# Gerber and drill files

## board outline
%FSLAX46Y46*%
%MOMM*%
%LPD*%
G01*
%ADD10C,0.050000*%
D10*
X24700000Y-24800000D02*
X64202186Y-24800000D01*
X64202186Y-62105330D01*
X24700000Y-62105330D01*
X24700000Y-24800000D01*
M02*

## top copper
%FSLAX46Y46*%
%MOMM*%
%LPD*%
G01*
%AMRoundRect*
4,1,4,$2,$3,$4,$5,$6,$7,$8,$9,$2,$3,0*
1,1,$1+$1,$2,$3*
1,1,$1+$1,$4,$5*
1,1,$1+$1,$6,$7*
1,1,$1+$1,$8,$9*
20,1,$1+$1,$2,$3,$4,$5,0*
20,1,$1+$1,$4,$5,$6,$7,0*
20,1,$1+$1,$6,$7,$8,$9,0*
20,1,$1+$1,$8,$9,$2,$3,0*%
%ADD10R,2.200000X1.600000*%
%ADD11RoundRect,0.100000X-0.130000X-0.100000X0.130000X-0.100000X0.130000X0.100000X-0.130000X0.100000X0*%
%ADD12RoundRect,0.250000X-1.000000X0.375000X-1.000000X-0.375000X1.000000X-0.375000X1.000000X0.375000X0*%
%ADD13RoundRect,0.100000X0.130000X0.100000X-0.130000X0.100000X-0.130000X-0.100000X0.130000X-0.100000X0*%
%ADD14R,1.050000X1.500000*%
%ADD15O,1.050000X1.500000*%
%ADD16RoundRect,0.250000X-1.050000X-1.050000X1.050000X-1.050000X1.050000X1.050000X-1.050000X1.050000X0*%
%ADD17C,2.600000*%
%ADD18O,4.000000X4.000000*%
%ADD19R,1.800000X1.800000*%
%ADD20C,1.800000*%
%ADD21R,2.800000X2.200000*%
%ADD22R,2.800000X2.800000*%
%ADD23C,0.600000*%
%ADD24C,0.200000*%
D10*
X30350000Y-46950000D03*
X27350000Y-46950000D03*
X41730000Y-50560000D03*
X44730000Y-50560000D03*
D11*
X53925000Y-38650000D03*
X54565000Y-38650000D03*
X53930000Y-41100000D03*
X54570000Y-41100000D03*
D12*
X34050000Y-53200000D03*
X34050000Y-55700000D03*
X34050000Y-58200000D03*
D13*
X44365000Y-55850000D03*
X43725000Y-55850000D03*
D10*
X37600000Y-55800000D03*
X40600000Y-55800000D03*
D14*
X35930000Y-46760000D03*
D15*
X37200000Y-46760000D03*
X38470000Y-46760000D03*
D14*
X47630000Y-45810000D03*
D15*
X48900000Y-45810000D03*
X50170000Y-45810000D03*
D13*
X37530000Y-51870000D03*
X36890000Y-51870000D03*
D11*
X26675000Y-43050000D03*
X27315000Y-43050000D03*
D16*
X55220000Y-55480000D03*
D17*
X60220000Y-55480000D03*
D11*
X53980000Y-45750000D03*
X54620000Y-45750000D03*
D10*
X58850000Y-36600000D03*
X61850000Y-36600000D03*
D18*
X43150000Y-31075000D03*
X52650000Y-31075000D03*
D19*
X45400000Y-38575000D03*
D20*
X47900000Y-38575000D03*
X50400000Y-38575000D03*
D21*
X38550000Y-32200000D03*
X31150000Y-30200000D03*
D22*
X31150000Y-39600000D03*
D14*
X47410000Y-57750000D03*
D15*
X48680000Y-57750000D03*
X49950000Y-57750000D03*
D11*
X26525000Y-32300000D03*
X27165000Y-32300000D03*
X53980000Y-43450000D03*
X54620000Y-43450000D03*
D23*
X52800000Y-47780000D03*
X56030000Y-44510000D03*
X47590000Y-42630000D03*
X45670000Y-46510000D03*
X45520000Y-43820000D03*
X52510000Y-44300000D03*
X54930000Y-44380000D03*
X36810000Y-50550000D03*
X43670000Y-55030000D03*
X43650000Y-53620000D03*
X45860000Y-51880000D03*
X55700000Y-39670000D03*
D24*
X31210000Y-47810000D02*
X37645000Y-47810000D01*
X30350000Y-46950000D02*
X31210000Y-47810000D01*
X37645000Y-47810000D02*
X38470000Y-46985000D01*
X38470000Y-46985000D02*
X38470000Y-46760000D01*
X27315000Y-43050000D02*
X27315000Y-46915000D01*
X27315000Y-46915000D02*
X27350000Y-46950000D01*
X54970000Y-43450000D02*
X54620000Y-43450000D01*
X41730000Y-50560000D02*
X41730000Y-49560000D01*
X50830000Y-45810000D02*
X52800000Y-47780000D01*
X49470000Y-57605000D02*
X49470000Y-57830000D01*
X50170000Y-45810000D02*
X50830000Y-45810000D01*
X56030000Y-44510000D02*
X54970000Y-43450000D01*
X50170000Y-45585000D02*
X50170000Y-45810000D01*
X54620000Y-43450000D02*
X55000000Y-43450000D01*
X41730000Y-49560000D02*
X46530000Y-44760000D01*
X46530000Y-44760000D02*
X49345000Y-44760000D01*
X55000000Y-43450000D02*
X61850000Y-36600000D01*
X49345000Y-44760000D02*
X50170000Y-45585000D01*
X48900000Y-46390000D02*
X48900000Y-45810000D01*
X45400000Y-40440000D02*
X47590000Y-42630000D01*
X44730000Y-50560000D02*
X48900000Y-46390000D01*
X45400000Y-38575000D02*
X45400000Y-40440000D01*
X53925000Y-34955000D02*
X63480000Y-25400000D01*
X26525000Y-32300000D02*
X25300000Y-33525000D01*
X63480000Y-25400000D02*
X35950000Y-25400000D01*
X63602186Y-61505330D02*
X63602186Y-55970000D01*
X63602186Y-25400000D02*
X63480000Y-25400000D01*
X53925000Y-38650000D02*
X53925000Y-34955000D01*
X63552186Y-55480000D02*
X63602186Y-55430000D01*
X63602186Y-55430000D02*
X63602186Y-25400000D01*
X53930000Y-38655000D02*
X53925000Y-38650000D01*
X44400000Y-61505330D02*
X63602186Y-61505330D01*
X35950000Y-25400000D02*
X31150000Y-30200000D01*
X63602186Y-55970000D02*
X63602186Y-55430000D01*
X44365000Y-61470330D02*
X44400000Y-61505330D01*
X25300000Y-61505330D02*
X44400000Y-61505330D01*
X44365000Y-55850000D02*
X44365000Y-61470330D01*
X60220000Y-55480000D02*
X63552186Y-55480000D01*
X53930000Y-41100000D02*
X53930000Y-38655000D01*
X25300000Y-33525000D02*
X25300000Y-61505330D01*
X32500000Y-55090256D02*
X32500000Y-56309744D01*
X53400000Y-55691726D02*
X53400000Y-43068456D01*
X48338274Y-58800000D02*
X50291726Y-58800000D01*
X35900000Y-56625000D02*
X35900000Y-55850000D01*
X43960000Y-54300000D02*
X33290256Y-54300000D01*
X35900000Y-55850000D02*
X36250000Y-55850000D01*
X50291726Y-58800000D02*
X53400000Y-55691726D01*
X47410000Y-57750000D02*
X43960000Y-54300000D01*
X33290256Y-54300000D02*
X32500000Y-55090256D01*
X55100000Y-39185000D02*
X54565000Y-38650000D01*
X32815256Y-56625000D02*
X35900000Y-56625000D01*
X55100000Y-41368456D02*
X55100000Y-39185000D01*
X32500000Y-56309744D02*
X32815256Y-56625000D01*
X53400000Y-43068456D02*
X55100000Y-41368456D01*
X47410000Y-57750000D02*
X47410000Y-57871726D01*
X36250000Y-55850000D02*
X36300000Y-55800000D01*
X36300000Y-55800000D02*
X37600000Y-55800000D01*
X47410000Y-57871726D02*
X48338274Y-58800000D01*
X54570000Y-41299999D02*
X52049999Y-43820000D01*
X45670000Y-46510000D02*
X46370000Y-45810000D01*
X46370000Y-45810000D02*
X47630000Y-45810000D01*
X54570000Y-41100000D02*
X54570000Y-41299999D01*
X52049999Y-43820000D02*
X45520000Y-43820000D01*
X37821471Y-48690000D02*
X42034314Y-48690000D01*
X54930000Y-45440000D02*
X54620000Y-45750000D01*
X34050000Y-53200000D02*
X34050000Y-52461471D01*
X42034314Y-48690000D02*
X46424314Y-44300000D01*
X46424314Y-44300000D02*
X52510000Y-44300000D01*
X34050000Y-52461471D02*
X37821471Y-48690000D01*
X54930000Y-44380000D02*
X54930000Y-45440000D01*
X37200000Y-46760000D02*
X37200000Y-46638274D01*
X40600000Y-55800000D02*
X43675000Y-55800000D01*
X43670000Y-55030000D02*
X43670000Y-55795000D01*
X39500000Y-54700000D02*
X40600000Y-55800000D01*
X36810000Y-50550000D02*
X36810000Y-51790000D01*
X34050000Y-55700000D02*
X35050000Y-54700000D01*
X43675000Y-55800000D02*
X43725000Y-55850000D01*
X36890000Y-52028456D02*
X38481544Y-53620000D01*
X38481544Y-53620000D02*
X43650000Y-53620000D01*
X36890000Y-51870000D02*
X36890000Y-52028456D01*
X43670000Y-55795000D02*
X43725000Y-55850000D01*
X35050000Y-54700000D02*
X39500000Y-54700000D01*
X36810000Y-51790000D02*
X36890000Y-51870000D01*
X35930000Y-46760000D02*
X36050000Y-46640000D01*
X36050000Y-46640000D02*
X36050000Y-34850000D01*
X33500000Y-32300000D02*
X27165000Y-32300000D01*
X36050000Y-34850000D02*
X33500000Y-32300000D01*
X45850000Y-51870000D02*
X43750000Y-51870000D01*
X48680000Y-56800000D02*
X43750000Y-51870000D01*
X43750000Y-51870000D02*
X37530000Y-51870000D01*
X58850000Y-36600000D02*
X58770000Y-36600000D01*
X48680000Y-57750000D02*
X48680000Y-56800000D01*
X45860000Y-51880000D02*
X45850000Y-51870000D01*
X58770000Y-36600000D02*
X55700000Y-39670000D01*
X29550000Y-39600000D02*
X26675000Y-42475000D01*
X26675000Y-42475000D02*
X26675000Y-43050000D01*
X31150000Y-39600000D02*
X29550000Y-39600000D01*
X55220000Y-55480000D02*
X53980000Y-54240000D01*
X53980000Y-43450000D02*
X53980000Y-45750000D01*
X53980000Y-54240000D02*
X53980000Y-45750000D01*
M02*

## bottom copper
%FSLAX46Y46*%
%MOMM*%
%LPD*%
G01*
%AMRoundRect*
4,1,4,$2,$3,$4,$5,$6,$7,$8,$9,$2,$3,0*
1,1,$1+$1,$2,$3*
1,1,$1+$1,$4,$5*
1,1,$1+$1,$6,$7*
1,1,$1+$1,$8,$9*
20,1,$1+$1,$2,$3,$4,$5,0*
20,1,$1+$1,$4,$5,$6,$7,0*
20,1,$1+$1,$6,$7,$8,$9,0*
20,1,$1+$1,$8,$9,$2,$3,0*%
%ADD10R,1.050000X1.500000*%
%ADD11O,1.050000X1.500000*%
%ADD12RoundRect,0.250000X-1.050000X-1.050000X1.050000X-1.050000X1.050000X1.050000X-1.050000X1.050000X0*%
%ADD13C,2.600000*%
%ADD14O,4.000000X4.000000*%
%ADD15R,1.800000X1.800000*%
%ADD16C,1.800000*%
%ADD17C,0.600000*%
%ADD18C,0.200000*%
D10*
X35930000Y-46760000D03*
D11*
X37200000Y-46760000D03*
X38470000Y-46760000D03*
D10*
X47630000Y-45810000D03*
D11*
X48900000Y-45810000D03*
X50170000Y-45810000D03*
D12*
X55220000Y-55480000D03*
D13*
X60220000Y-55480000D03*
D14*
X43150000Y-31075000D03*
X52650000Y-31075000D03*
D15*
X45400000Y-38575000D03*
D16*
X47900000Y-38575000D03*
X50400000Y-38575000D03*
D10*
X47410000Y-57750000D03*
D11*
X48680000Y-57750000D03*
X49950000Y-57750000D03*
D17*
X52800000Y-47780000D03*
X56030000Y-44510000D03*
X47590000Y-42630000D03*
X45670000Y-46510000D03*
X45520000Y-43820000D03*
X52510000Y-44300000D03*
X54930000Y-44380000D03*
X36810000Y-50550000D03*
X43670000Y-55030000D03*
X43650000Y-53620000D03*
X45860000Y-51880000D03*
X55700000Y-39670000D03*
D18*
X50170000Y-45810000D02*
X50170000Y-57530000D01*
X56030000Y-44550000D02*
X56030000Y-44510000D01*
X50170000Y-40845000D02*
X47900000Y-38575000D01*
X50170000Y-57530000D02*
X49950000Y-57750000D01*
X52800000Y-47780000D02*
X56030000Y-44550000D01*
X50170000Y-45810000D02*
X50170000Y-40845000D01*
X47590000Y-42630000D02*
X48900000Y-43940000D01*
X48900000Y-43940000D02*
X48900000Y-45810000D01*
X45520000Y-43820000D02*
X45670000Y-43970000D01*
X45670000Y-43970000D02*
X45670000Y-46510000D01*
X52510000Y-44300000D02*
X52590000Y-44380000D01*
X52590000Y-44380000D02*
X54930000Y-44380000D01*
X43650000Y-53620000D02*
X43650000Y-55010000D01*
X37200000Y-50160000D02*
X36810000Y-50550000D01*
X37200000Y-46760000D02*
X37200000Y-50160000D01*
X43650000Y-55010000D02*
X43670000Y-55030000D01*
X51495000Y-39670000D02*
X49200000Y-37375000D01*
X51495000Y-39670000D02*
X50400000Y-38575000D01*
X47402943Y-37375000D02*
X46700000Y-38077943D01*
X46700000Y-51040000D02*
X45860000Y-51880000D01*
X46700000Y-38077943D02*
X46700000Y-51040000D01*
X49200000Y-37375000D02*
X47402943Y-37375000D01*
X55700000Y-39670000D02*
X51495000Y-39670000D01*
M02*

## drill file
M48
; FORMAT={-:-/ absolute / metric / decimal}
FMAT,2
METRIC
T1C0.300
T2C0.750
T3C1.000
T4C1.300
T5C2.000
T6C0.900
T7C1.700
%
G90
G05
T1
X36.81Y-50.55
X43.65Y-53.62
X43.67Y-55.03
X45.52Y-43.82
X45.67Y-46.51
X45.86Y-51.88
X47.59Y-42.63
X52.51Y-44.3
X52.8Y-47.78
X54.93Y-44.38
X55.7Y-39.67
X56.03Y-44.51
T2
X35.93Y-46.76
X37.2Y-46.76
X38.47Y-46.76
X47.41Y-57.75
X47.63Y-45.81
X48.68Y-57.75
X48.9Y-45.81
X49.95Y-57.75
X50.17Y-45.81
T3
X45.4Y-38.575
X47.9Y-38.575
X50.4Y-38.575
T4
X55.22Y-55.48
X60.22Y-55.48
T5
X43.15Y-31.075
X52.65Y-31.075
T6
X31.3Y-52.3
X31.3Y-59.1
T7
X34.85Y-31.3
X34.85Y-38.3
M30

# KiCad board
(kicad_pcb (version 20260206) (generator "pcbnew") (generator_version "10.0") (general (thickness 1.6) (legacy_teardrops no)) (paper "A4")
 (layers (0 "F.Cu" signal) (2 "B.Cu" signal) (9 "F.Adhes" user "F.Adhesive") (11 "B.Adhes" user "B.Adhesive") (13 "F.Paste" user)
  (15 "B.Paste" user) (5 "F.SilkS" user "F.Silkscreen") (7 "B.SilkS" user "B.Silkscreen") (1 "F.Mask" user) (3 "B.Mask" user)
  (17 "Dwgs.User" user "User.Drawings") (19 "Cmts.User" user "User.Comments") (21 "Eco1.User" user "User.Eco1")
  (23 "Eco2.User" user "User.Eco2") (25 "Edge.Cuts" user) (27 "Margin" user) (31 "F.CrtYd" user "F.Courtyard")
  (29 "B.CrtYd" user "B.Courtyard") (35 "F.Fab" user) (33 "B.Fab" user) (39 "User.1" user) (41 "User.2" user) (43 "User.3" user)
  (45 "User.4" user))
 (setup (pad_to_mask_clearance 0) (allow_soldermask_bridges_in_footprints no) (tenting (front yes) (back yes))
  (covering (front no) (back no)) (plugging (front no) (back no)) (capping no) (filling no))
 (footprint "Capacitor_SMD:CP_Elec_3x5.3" (layer "F.Cu") (at 28.85 46.95 180)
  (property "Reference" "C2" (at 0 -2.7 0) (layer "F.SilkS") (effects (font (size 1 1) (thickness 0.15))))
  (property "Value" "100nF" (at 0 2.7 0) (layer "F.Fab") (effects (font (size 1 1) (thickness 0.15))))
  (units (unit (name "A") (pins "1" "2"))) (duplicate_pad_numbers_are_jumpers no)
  (pad "1" smd rect (at -1.5 0 180) (size 2.2 1.6) (layers "F.Cu" "F.Mask" "F.Paste") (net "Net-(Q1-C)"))
  (pad "2" smd rect (at 1.5 0 180) (size 2.2 1.6) (layers "F.Cu" "F.Mask" "F.Paste") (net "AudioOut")))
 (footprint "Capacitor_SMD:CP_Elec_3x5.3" (layer "F.Cu") (at 43.23 50.56)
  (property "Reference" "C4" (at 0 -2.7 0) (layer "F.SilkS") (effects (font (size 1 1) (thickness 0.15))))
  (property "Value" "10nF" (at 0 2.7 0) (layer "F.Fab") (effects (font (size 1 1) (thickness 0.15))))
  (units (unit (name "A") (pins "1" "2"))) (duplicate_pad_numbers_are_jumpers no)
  (pad "1" smd rect (at -1.5 0) (size 2.2 1.6) (layers "F.Cu" "F.Mask" "F.Paste") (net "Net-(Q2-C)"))
  (pad "2" smd rect (at 1.5 0) (size 2.2 1.6) (layers "F.Cu" "F.Mask" "F.Paste") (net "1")))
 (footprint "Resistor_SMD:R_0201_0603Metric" (layer "F.Cu") (at 54.245 38.65)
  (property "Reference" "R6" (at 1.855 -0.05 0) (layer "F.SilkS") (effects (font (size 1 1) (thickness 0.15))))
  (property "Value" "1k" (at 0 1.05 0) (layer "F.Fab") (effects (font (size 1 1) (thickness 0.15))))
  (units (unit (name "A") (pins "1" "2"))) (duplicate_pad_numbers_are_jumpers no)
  (pad "" smd roundrect (at -0.345 0) (size 0.318 0.36) (layers "F.Paste") (roundrect_rratio 0.25))
  (pad "" smd roundrect (at 0.345 0) (size 0.318 0.36) (layers "F.Paste") (roundrect_rratio 0.25))
  (pad "1" smd roundrect (at -0.32 0) (size 0.46 0.4) (layers "F.Cu" "F.Mask") (roundrect_rratio 0.25) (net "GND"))
  (pad "2" smd roundrect (at 0.32 0) (size 0.46 0.4) (layers "F.Cu" "F.Mask") (roundrect_rratio 0.25) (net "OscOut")))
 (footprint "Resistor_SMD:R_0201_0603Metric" (layer "F.Cu") (at 54.25 41.1)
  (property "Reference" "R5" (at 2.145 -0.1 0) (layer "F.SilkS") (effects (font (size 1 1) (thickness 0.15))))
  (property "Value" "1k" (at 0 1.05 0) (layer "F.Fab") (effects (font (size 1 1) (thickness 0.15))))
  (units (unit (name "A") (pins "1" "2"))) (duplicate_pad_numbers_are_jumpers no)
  (pad "" smd roundrect (at -0.345 0) (size 0.318 0.36) (layers "F.Paste") (roundrect_rratio 0.25))
  (pad "" smd roundrect (at 0.345 0) (size 0.318 0.36) (layers "F.Paste") (roundrect_rratio 0.25))
  (pad "1" smd roundrect (at -0.32 0) (size 0.46 0.4) (layers "F.Cu" "F.Mask") (roundrect_rratio 0.25) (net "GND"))
  (pad "2" smd roundrect (at 0.32 0) (size 0.46 0.4) (layers "F.Cu" "F.Mask") (roundrect_rratio 0.25) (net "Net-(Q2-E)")))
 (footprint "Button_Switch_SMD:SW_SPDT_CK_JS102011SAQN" (layer "F.Cu") (at 31.3 55.7 -90)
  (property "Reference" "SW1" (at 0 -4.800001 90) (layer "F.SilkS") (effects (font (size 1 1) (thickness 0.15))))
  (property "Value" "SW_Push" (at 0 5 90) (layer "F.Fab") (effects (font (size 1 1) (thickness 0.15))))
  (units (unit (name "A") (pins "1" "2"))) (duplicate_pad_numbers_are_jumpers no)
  (pad "" np_thru_hole circle (at -3.4 0 270) (size 0.9 0.9) (drill 0.9) (layers "*.Cu" "*.Mask"))
  (pad "" np_thru_hole circle (at 3.4 0 270) (size 0.9 0.9) (drill 0.9) (layers "*.Cu" "*.Mask"))
  (pad "1" smd roundrect (at -2.5 -2.75 270) (size 1.25 2.5) (layers "F.Cu" "F.Mask" "F.Paste") (roundrect_rratio 0.2) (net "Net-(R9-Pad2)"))
  (pad "2" smd roundrect (at 0 -2.75 270) (size 1.25 2.5) (layers "F.Cu" "F.Mask" "F.Paste") (roundrect_rratio 0.2) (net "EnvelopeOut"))
  (pad "3" smd roundrect (at 2.5 -2.75 270) (size 1.25 2.5) (layers "F.Cu" "F.Mask" "F.Paste") (roundrect_rratio 0.2)))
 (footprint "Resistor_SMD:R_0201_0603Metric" (layer "F.Cu") (at 44.045 55.85 180)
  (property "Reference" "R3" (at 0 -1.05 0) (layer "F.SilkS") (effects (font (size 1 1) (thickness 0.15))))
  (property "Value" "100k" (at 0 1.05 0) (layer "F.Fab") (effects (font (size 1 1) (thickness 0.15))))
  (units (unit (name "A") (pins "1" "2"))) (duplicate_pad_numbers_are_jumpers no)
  (pad "" smd roundrect (at -0.345 0 180) (size 0.318 0.36) (layers "F.Paste") (roundrect_rratio 0.25))
  (pad "" smd roundrect (at 0.345 0 180) (size 0.318 0.36) (layers "F.Paste") (roundrect_rratio 0.25))
  (pad "1" smd roundrect (at -0.32 0 180) (size 0.46 0.4) (layers "F.Cu" "F.Mask") (roundrect_rratio 0.25) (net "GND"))
  (pad "2" smd roundrect (at 0.32 0 180) (size 0.46 0.4) (layers "F.Cu" "F.Mask") (roundrect_rratio 0.25) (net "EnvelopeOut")))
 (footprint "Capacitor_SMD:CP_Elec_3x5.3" (layer "F.Cu") (at 39.1 55.8)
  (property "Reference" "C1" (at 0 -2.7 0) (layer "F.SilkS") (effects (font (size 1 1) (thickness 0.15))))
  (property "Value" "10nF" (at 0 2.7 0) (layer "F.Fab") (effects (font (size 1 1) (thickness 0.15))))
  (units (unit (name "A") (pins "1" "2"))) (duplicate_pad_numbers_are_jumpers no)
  (pad "1" smd rect (at -1.5 0) (size 2.2 1.6) (layers "F.Cu" "F.Mask" "F.Paste") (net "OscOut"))
  (pad "2" smd rect (at 1.5 0) (size 2.2 1.6) (layers "F.Cu" "F.Mask" "F.Paste") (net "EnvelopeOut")))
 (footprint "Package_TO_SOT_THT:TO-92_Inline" (layer "F.Cu") (at 35.93 46.76)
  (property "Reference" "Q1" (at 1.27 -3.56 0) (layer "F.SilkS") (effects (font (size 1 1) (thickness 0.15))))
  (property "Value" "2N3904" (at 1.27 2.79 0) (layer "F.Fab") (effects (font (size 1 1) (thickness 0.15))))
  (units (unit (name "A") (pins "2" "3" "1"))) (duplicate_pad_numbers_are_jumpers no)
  (pad "1" thru_hole rect (at 0 0) (size 1.05 1.5) (drill 0.75) (layers "*.Cu" "*.Mask") (remove_unused_layers no) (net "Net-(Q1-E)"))
  (pad "2" thru_hole oval (at 1.27 0) (size 1.05 1.5) (drill 0.75) (layers "*.Cu" "*.Mask") (remove_unused_layers no) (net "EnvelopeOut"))
  (pad "3" thru_hole oval (at 2.54 0) (size 1.05 1.5) (drill 0.75) (layers "*.Cu" "*.Mask") (remove_unused_layers no) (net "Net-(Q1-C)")))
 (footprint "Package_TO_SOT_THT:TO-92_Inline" (layer "F.Cu") (at 47.63 45.81)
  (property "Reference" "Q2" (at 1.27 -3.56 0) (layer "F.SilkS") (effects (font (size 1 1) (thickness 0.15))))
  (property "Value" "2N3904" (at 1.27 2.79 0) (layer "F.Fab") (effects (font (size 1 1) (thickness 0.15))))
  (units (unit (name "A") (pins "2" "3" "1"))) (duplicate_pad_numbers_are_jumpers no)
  (pad "1" thru_hole rect (at 0 0) (size 1.05 1.5) (drill 0.75) (layers "*.Cu" "*.Mask") (remove_unused_layers no) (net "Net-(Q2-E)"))
  (pad "2" thru_hole oval (at 1.27 0) (size 1.05 1.5) (drill 0.75) (layers "*.Cu" "*.Mask") (remove_unused_layers no) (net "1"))
  (pad "3" thru_hole oval (at 2.54 0) (size 1.05 1.5) (drill 0.75) (layers "*.Cu" "*.Mask") (remove_unused_layers no) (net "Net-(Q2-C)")))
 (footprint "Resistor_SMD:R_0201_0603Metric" (layer "F.Cu") (at 37.21 51.87 180)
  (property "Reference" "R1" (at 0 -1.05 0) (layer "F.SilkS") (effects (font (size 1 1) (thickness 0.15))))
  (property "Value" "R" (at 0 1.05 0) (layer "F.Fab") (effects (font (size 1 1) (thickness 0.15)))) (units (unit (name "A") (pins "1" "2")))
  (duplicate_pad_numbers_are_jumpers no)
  (pad "" smd roundrect (at -0.345 0 180) (size 0.318 0.36) (layers "F.Paste") (roundrect_rratio 0.25))
  (pad "" smd roundrect (at 0.345 0 180) (size 0.318 0.36) (layers "F.Paste") (roundrect_rratio 0.25))
  (pad "1" smd roundrect (at -0.32 0 180) (size 0.46 0.4) (layers "F.Cu" "F.Mask") (roundrect_rratio 0.25) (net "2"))
  (pad "2" smd roundrect (at 0.32 0 180) (size 0.46 0.4) (layers "F.Cu" "F.Mask") (roundrect_rratio 0.25) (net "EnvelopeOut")))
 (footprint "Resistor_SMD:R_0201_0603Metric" (layer "F.Cu") (at 26.995 43.05)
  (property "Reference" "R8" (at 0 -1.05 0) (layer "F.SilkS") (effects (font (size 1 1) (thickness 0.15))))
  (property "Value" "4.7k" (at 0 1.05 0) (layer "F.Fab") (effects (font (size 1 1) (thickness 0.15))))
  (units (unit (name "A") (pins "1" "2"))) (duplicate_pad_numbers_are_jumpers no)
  (pad "" smd roundrect (at -0.345 0) (size 0.318 0.36) (layers "F.Paste") (roundrect_rratio 0.25))
  (pad "" smd roundrect (at 0.345 0) (size 0.318 0.36) (layers "F.Paste") (roundrect_rratio 0.25))
  (pad "1" smd roundrect (at -0.32 0) (size 0.46 0.4) (layers "F.Cu" "F.Mask") (roundrect_rratio 0.25) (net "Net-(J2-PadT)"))
  (pad "2" smd roundrect (at 0.32 0) (size 0.46 0.4) (layers "F.Cu" "F.Mask") (roundrect_rratio 0.25) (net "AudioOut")))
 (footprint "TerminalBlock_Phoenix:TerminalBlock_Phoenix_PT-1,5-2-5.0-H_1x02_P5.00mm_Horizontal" (layer "F.Cu") (at 55.22 55.48)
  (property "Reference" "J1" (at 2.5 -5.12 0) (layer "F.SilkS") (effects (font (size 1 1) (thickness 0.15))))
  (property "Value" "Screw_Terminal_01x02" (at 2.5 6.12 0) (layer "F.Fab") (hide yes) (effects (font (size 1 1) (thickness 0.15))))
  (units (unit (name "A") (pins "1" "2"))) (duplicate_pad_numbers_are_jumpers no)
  (pad "1" thru_hole roundrect (at 0 0) (size 2.6 2.6) (drill 1.3) (layers "*.Cu" "*.Mask") (remove_unused_layers no)
   (roundrect_rratio 0.096154) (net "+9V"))
  (pad "2" thru_hole circle (at 5 0) (size 2.6 2.6) (drill 1.3) (layers "*.Cu" "*.Mask") (remove_unused_layers no) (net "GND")))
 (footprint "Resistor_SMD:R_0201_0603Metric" (layer "F.Cu") (at 54.3 45.75)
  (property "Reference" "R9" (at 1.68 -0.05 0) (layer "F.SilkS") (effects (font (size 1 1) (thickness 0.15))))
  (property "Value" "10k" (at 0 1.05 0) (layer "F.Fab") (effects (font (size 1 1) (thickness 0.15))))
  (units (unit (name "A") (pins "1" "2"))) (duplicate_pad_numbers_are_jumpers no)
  (pad "" smd roundrect (at -0.345 0) (size 0.318 0.36) (layers "F.Paste") (roundrect_rratio 0.25))
  (pad "" smd roundrect (at 0.345 0) (size 0.318 0.36) (layers "F.Paste") (roundrect_rratio 0.25))
  (pad "1" smd roundrect (at -0.32 0) (size 0.46 0.4) (layers "F.Cu" "F.Mask") (roundrect_rratio 0.25) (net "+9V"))
  (pad "2" smd roundrect (at 0.32 0) (size 0.46 0.4) (layers "F.Cu" "F.Mask") (roundrect_rratio 0.25) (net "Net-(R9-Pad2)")))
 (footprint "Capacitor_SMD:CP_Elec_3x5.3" (layer "F.Cu") (at 60.35 36.6)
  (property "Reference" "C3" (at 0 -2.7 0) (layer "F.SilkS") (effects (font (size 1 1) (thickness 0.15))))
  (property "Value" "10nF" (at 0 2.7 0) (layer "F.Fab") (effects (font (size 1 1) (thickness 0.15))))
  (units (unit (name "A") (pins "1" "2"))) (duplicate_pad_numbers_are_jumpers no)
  (pad "1" smd rect (at -1.5 0) (size 2.2 1.6) (layers "F.Cu" "F.Mask" "F.Paste") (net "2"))
  (pad "2" smd rect (at 1.5 0) (size 2.2 1.6) (layers "F.Cu" "F.Mask" "F.Paste") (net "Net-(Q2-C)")))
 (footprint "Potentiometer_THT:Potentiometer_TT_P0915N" (layer "F.Cu") (at 45.4 38.575)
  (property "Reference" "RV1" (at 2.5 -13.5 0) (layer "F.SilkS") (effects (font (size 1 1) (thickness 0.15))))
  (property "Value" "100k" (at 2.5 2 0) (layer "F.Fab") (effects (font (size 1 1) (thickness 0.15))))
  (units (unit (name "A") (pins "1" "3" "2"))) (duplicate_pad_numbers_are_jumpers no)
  (pad "" thru_hole oval (at -2.25 -7.5) (size 4 4) (drill 2) (layers "*.Cu" "*.Mask") (remove_unused_layers no))
  (pad "" thru_hole oval (at 7.25 -7.5) (size 4 4) (drill 2) (layers "*.Cu" "*.Mask") (remove_unused_layers no))
  (pad "1" thru_hole rect (at 0 0) (size 1.8 1.8) (drill 1) (layers "*.Cu" "*.Mask") (remove_unused_layers no) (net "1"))
  (pad "2" thru_hole circle (at 2.5 0) (size 1.8 1.8) (drill 1) (layers "*.Cu" "*.Mask") (remove_unused_layers no) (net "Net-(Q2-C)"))
  (pad "3" thru_hole circle (at 5 0) (size 1.8 1.8) (drill 1) (layers "*.Cu" "*.Mask") (remove_unused_layers no) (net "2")))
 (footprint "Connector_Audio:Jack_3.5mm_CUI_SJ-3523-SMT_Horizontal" (layer "F.Cu") (at 34.85 33.8)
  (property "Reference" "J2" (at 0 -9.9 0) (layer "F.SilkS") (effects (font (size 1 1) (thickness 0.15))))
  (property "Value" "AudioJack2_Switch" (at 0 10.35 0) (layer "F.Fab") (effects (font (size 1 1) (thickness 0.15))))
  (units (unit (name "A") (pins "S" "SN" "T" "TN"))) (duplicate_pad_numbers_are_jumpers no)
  (pad "" np_thru_hole circle (at 0 -2.5) (size 1.7 1.7) (drill 1.7) (layers "*.Cu" "*.Mask"))
  (pad "" np_thru_hole circle (at 0 4.5) (size 1.7 1.7) (drill 1.7) (layers "*.Cu" "*.Mask"))
  (pad "R" smd rect (at 3.7 -1.6) (size 2.8 2.2) (layers "F.Cu" "F.Mask" "F.Paste"))
  (pad "S" smd rect (at -3.7 -3.6) (size 2.8 2.2) (layers "F.Cu" "F.Mask" "F.Paste") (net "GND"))
  (pad "T" smd rect (at -3.7 5.8) (size 2.8 2.8) (layers "F.Cu" "F.Mask" "F.Paste") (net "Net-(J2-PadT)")))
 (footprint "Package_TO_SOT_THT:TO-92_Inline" (layer "F.Cu") (at 47.41 57.75)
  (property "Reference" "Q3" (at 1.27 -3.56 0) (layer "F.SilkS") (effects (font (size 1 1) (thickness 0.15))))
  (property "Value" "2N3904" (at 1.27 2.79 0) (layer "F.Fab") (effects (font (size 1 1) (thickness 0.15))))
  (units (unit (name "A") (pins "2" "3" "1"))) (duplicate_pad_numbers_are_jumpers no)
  (pad "1" thru_hole rect (at 0 0) (size 1.05 1.5) (drill 0.75) (layers "*.Cu" "*.Mask") (remove_unused_layers no) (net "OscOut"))
  (pad "2" thru_hole oval (at 1.27 0) (size 1.05 1.5) (drill 0.75) (layers "*.Cu" "*.Mask") (remove_unused_layers no) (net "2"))
  (pad "3" thru_hole oval (at 2.54 0) (size 1.05 1.5) (drill 0.75) (layers "*.Cu" "*.Mask") (remove_unused_layers no) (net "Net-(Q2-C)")))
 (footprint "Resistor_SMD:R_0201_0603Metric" (layer "F.Cu") (at 26.845 32.3)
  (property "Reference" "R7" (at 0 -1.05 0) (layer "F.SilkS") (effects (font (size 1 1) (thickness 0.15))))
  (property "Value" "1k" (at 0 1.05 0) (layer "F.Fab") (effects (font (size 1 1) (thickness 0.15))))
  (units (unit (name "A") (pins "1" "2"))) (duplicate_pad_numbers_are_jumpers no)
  (pad "" smd roundrect (at -0.345 0) (size 0.318 0.36) (layers "F.Paste") (roundrect_rratio 0.25))
  (pad "" smd roundrect (at 0.345 0) (size 0.318 0.36) (layers "F.Paste") (roundrect_rratio 0.25))
  (pad "1" smd roundrect (at -0.32 0) (size 0.46 0.4) (layers "F.Cu" "F.Mask") (roundrect_rratio 0.25) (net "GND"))
  (pad "2" smd roundrect (at 0.32 0) (size 0.46 0.4) (layers "F.Cu" "F.Mask") (roundrect_rratio 0.25) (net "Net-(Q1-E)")))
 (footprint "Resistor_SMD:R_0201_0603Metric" (layer "F.Cu") (at 54.3 43.45)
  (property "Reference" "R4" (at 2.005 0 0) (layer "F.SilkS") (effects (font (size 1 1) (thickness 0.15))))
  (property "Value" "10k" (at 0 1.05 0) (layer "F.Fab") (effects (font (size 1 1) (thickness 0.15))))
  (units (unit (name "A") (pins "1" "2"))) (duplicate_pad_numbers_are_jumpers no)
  (pad "" smd roundrect (at -0.345 0) (size 0.318 0.36) (layers "F.Paste") (roundrect_rratio 0.25))
  (pad "" smd roundrect (at 0.345 0) (size 0.318 0.36) (layers "F.Paste") (roundrect_rratio 0.25))
  (pad "1" smd roundrect (at -0.32 0) (size 0.46 0.4) (layers "F.Cu" "F.Mask") (roundrect_rratio 0.25) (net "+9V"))
  (pad "2" smd roundrect (at 0.32 0) (size 0.46 0.4) (layers "F.Cu" "F.Mask") (roundrect_rratio 0.25) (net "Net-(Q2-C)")))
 (gr_rect (start 24.7 24.8) (end 64.202186 62.10533) (stroke (width 0.05) (type default)) (fill no) (layer "Edge.Cuts"))
 (segment (start 31.21 47.81) (end 37.645 47.81) (width 0.2) (layer "F.Cu") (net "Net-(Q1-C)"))
 (segment (start 30.35 46.95) (end 31.21 47.81) (width 0.2) (layer "F.Cu") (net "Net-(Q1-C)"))
 (segment (start 37.645 47.81) (end 38.47 46.985) (width 0.2) (layer "F.Cu") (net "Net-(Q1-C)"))
 (segment (start 38.47 46.985) (end 38.47 46.76) (width 0.2) (layer "F.Cu") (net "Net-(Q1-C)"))
 (segment (start 27.315 43.05) (end 27.315 46.915) (width 0.2) (layer "F.Cu") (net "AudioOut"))
 (segment (start 27.315 46.915) (end 27.35 46.95) (width 0.2) (layer "F.Cu") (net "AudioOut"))
 (segment (start 54.97 43.45) (end 54.62 43.45) (width 0.2) (layer "F.Cu") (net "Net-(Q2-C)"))
 (segment (start 41.73 50.56) (end 41.73 49.56) (width 0.2) (layer "F.Cu") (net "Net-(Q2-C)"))
 (segment (start 50.83 45.81) (end 52.8 47.78) (width 0.2) (layer "F.Cu") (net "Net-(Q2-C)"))
 (segment (start 49.47 57.605) (end 49.47 57.83) (width 0.2) (layer "F.Cu") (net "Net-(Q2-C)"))
 (segment (start 50.17 45.81) (end 50.83 45.81) (width 0.2) (layer "F.Cu") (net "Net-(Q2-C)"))
 (segment (start 56.03 44.51) (end 54.97 43.45) (width 0.2) (layer "F.Cu") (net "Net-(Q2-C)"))
 (segment (start 50.17 45.585) (end 50.17 45.81) (width 0.2) (layer "F.Cu") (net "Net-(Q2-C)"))
 (segment (start 54.62 43.45) (end 55 43.45) (width 0.2) (layer "F.Cu") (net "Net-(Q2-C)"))
 (segment (start 41.73 49.56) (end 46.53 44.76) (width 0.2) (layer "F.Cu") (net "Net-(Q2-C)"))
 (segment (start 46.53 44.76) (end 49.345 44.76) (width 0.2) (layer "F.Cu") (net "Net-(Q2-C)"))
 (segment (start 55 43.45) (end 61.85 36.6) (width 0.2) (layer "F.Cu") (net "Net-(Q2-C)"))
 (segment (start 49.345 44.76) (end 50.17 45.585) (width 0.2) (layer "F.Cu") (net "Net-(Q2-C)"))
 (via (at 52.8 47.78) (size 0.6) (drill 0.3) (layers "F.Cu" "B.Cu") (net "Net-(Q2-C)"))
 (via (at 56.03 44.51) (size 0.6) (drill 0.3) (layers "F.Cu" "B.Cu") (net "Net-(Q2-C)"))
 (segment (start 50.17 45.81) (end 50.17 57.53) (width 0.2) (layer "B.Cu") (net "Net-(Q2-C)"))
 (segment (start 56.03 44.55) (end 56.03 44.51) (width 0.2) (layer "B.Cu") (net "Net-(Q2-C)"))
 (segment (start 50.17 40.845) (end 47.9 38.575) (width 0.2) (layer "B.Cu") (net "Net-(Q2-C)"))
 (segment (start 50.17 57.53) (end 49.95 57.75) (width 0.2) (layer "B.Cu") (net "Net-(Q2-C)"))
 (segment (start 52.8 47.78) (end 56.03 44.55) (width 0.2) (layer "B.Cu") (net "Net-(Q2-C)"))
 (segment (start 50.17 45.81) (end 50.17 40.845) (width 0.2) (layer "B.Cu") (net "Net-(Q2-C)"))
 (segment (start 48.9 46.39) (end 48.9 45.81) (width 0.2) (layer "F.Cu") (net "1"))
 (segment (start 45.4 40.44) (end 47.59 42.63) (width 0.2) (layer "F.Cu") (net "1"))
 (segment (start 44.73 50.56) (end 48.9 46.39) (width 0.2) (layer "F.Cu") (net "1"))
 (segment (start 45.4 38.575) (end 45.4 40.44) (width 0.2) (layer "F.Cu") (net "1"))
 (via (at 47.59 42.63) (size 0.6) (drill 0.3) (layers "F.Cu" "B.Cu") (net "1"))
 (segment (start 47.59 42.63) (end 48.9 43.94) (width 0.2) (layer "B.Cu") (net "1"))
 (segment (start 48.9 43.94) (end 48.9 45.81) (width 0.2) (layer "B.Cu") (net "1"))
 (segment (start 53.925 34.955) (end 63.48 25.4) (width 0.2) (layer "F.Cu") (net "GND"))
 (segment (start 26.525 32.3) (end 25.3 33.525) (width 0.2) (layer "F.Cu") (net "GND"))
 (segment (start 63.48 25.4) (end 35.95 25.4) (width 0.2) (layer "F.Cu") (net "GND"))
 (segment (start 63.602186 61.50533) (end 63.602186 55.97) (width 0.2) (layer "F.Cu") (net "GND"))
 (segment (start 63.602186 25.4) (end 63.48 25.4) (width 0.2) (layer "F.Cu") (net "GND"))
 (segment (start 53.925 38.65) (end 53.925 34.955) (width 0.2) (layer "F.Cu") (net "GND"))
 (segment (start 63.552186 55.48) (end 63.602186 55.43) (width 0.2) (layer "F.Cu") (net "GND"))
 (segment (start 63.602186 55.43) (end 63.602186 25.4) (width 0.2) (layer "F.Cu") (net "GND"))
 (segment (start 53.93 38.655) (end 53.925 38.65) (width 0.2) (layer "F.Cu") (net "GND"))
 (segment (start 44.4 61.50533) (end 63.602186 61.50533) (width 0.2) (layer "F.Cu") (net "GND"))
 (segment (start 35.95 25.4) (end 31.15 30.2) (width 0.2) (layer "F.Cu") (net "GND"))
 (segment (start 63.602186 55.97) (end 63.602186 55.43) (width 0.2) (layer "F.Cu") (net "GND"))
 (segment (start 44.365 61.47033) (end 44.4 61.50533) (width 0.2) (layer "F.Cu") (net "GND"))
 (segment (start 25.3 61.50533) (end 44.4 61.50533) (width 0.2) (layer "F.Cu") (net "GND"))
 (segment (start 44.365 55.85) (end 44.365 61.47033) (width 0.2) (layer "F.Cu") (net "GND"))
 (segment (start 60.22 55.48) (end 63.552186 55.48) (width 0.2) (layer "F.Cu") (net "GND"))
 (segment (start 53.93 41.1) (end 53.93 38.655) (width 0.2) (layer "F.Cu") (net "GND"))
 (segment (start 25.3 33.525) (end 25.3 61.50533) (width 0.2) (layer "F.Cu") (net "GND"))
 (segment (start 32.5 55.090256) (end 32.5 56.309744) (width 0.2) (layer "F.Cu") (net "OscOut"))
 (segment (start 53.4 55.691726) (end 53.4 43.068456) (width 0.2) (layer "F.Cu") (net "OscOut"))
 (segment (start 48.338274 58.8) (end 50.291726 58.8) (width 0.2) (layer "F.Cu") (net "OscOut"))
 (segment (start 35.9 56.625) (end 35.9 55.85) (width 0.2) (layer "F.Cu") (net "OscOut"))
 (segment (start 43.96 54.3) (end 33.290256 54.3) (width 0.2) (layer "F.Cu") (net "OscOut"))
 (segment (start 35.9 55.85) (end 36.25 55.85) (width 0.2) (layer "F.Cu") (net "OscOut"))
 (segment (start 50.291726 58.8) (end 53.4 55.691726) (width 0.2) (layer "F.Cu") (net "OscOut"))
 (segment (start 47.41 57.75) (end 43.96 54.3) (width 0.2) (layer "F.Cu") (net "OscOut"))
 (segment (start 33.290256 54.3) (end 32.5 55.090256) (width 0.2) (layer "F.Cu") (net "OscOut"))
 (segment (start 55.1 39.185) (end 54.565 38.65) (width 0.2) (layer "F.Cu") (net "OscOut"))
 (segment (start 32.815256 56.625) (end 35.9 56.625) (width 0.2) (layer "F.Cu") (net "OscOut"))
 (segment (start 55.1 41.368456) (end 55.1 39.185) (width 0.2) (layer "F.Cu") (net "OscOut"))
 (segment (start 32.5 56.309744) (end 32.815256 56.625) (width 0.2) (layer "F.Cu") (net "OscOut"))
 (segment (start 53.4 43.068456) (end 55.1 41.368456) (width 0.2) (layer "F.Cu") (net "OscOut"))
 (segment (start 47.41 57.75) (end 47.41 57.871726) (width 0.2) (layer "F.Cu") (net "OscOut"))
 (segment (start 36.25 55.85) (end 36.3 55.8) (width 0.2) (layer "F.Cu") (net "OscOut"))
 (segment (start 36.3 55.8) (end 37.6 55.8) (width 0.2) (layer "F.Cu") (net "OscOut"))
 (segment (start 47.41 57.871726) (end 48.338274 58.8) (width 0.2) (layer "F.Cu") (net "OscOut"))
 (segment (start 54.57 41.299999) (end 52.049999 43.82) (width 0.2) (layer "F.Cu") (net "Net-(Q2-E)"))
 (segment (start 45.67 46.51) (end 46.37 45.81) (width 0.2) (layer "F.Cu") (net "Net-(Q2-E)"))
 (segment (start 46.37 45.81) (end 47.63 45.81) (width 0.2) (layer "F.Cu") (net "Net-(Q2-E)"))
 (segment (start 54.57 41.1) (end 54.57 41.299999) (width 0.2) (layer "F.Cu") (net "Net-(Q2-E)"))
 (segment (start 52.049999 43.82) (end 45.52 43.82) (width 0.2) (layer "F.Cu") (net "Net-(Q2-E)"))
 (via (at 45.67 46.51) (size 0.6) (drill 0.3) (layers "F.Cu" "B.Cu") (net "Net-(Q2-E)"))
 (via (at 45.52 43.82) (size 0.6) (drill 0.3) (layers "F.Cu" "B.Cu") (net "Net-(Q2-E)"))
 (segment (start 45.52 43.82) (end 45.67 43.97) (width 0.2) (layer "B.Cu") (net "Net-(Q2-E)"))
 (segment (start 45.67 43.97) (end 45.67 46.51) (width 0.2) (layer "B.Cu") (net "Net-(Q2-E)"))
 (segment (start 37.821471 48.69) (end 42.034314 48.69) (width 0.2) (layer "F.Cu") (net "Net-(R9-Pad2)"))
 (segment (start 54.93 45.44) (end 54.62 45.75) (width 0.2) (layer "F.Cu") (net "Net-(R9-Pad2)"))
 (segment (start 34.05 53.2) (end 34.05 52.461471) (width 0.2) (layer "F.Cu") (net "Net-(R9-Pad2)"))
 (segment (start 42.034314 48.69) (end 46.424314 44.3) (width 0.2) (layer "F.Cu") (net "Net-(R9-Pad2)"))
 (segment (start 46.424314 44.3) (end 52.51 44.3) (width 0.2) (layer "F.Cu") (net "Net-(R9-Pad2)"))
 (segment (start 34.05 52.461471) (end 37.821471 48.69) (width 0.2) (layer "F.Cu") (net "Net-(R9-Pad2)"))
 (segment (start 54.93 44.38) (end 54.93 45.44) (width 0.2) (layer "F.Cu") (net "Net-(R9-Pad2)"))
 (via (at 52.51 44.3) (size 0.6) (drill 0.3) (layers "F.Cu" "B.Cu") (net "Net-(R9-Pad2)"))
 (via (at 54.93 44.38) (size 0.6) (drill 0.3) (layers "F.Cu" "B.Cu") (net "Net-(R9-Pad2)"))
 (segment (start 52.51 44.3) (end 52.59 44.38) (width 0.2) (layer "B.Cu") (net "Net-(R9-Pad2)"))
 (segment (start 52.59 44.38) (end 54.93 44.38) (width 0.2) (layer "B.Cu") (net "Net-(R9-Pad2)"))
 (segment (start 37.2 46.76) (end 37.2 46.638274) (width 0.2) (layer "F.Cu") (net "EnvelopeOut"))
 (segment (start 40.6 55.8) (end 43.675 55.8) (width 0.2) (layer "F.Cu") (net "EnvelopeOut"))
 (segment (start 43.67 55.03) (end 43.67 55.795) (width 0.2) (layer "F.Cu") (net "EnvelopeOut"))
 (segment (start 39.5 54.7) (end 40.6 55.8) (width 0.2) (layer "F.Cu") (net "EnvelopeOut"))
 (segment (start 36.81 50.55) (end 36.81 51.79) (width 0.2) (layer "F.Cu") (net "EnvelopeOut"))
 (segment (start 34.05 55.7) (end 35.05 54.7) (width 0.2) (layer "F.Cu") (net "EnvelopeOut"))
 (segment (start 43.675 55.8) (end 43.725 55.85) (width 0.2) (layer "F.Cu") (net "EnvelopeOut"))
 (segment (start 36.89 52.028456) (end 38.481544 53.62) (width 0.2) (layer "F.Cu") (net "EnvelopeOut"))
 (segment (start 38.481544 53.62) (end 43.65 53.62) (width 0.2) (layer "F.Cu") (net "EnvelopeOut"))
 (segment (start 36.89 51.87) (end 36.89 52.028456) (width 0.2) (layer "F.Cu") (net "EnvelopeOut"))
 (segment (start 43.67 55.795) (end 43.725 55.85) (width 0.2) (layer "F.Cu") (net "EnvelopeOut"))
 (segment (start 35.05 54.7) (end 39.5 54.7) (width 0.2) (layer "F.Cu") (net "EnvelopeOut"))
 (segment (start 36.81 51.79) (end 36.89 51.87) (width 0.2) (layer "F.Cu") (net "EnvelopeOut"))
 (via (at 36.81 50.55) (size 0.6) (drill 0.3) (layers "F.Cu" "B.Cu") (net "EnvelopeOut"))
 (via (at 43.67 55.03) (size 0.6) (drill 0.3) (layers "F.Cu" "B.Cu") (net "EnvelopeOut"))
 (via (at 43.65 53.62) (size 0.6) (drill 0.3) (layers "F.Cu" "B.Cu") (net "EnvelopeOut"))
 (segment (start 43.65 53.62) (end 43.65 55.01) (width 0.2) (layer "B.Cu") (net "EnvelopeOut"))
 (segment (start 37.2 50.16) (end 36.81 50.55) (width 0.2) (layer "B.Cu") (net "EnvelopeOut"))
 (segment (start 37.2 46.76) (end 37.2 50.16) (width 0.2) (layer "B.Cu") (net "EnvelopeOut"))
 (segment (start 43.65 55.01) (end 43.67 55.03) (width 0.2) (layer "B.Cu") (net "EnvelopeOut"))
 (segment (start 35.93 46.76) (end 36.05 46.64) (width 0.2) (layer "F.Cu") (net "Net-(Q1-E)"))
 (segment (start 36.05 46.64) (end 36.05 34.85) (width 0.2) (layer "F.Cu") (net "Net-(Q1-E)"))
 (segment (start 33.5 32.3) (end 27.165 32.3) (width 0.2) (layer "F.Cu") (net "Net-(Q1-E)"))
 (segment (start 36.05 34.85) (end 33.5 32.3) (width 0.2) (layer "F.Cu") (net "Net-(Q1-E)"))
 (segment (start 45.85 51.87) (end 43.75 51.87) (width 0.2) (layer "F.Cu") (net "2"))
 (segment (start 48.68 56.8) (end 43.75 51.87) (width 0.2) (layer "F.Cu") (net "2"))
 (segment (start 43.75 51.87) (end 37.53 51.87) (width 0.2) (layer "F.Cu") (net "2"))
 (segment (start 58.85 36.6) (end 58.77 36.6) (width 0.2) (layer "F.Cu") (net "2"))
 (segment (start 48.68 57.75) (end 48.68 56.8) (width 0.2) (layer "F.Cu") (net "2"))
 (segment (start 45.86 51.88) (end 45.85 51.87) (width 0.2) (layer "F.Cu") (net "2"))
 (segment (start 58.77 36.6) (end 55.7 39.67) (width 0.2) (layer "F.Cu") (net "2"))
 (via (at 45.86 51.88) (size 0.6) (drill 0.3) (layers "F.Cu" "B.Cu") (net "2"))
 (via (at 55.7 39.67) (size 0.6) (drill 0.3) (layers "F.Cu" "B.Cu") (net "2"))
 (segment (start 51.495 39.67) (end 49.2 37.375) (width 0.2) (layer "B.Cu") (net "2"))
 (segment (start 51.495 39.67) (end 50.4 38.575) (width 0.2) (layer "B.Cu") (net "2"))
 (segment (start 47.402943 37.375) (end 46.7 38.077943) (width 0.2) (layer "B.Cu") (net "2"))
 (segment (start 46.7 51.04) (end 45.86 51.88) (width 0.2) (layer "B.Cu") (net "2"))
 (segment (start 46.7 38.077943) (end 46.7 51.04) (width 0.2) (layer "B.Cu") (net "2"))
 (segment (start 49.2 37.375) (end 47.402943 37.375) (width 0.2) (layer "B.Cu") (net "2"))
 (segment (start 55.7 39.67) (end 51.495 39.67) (width 0.2) (layer "B.Cu") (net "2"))
 (segment (start 29.55 39.6) (end 26.675 42.475) (width 0.2) (layer "F.Cu") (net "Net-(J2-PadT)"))
 (segment (start 26.675 42.475) (end 26.675 43.05) (width 0.2) (layer "F.Cu") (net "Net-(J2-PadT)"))
 (segment (start 31.15 39.6) (end 29.55 39.6) (width 0.2) (layer "F.Cu") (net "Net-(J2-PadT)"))
 (segment (start 55.22 55.48) (end 53.98 54.24) (width 0.2) (layer "F.Cu") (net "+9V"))
 (segment (start 53.98 43.45) (end 53.98 45.75) (width 0.2) (layer "F.Cu") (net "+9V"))
 (segment (start 53.98 54.24) (end 53.98 45.75) (width 0.2) (layer "F.Cu") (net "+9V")))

